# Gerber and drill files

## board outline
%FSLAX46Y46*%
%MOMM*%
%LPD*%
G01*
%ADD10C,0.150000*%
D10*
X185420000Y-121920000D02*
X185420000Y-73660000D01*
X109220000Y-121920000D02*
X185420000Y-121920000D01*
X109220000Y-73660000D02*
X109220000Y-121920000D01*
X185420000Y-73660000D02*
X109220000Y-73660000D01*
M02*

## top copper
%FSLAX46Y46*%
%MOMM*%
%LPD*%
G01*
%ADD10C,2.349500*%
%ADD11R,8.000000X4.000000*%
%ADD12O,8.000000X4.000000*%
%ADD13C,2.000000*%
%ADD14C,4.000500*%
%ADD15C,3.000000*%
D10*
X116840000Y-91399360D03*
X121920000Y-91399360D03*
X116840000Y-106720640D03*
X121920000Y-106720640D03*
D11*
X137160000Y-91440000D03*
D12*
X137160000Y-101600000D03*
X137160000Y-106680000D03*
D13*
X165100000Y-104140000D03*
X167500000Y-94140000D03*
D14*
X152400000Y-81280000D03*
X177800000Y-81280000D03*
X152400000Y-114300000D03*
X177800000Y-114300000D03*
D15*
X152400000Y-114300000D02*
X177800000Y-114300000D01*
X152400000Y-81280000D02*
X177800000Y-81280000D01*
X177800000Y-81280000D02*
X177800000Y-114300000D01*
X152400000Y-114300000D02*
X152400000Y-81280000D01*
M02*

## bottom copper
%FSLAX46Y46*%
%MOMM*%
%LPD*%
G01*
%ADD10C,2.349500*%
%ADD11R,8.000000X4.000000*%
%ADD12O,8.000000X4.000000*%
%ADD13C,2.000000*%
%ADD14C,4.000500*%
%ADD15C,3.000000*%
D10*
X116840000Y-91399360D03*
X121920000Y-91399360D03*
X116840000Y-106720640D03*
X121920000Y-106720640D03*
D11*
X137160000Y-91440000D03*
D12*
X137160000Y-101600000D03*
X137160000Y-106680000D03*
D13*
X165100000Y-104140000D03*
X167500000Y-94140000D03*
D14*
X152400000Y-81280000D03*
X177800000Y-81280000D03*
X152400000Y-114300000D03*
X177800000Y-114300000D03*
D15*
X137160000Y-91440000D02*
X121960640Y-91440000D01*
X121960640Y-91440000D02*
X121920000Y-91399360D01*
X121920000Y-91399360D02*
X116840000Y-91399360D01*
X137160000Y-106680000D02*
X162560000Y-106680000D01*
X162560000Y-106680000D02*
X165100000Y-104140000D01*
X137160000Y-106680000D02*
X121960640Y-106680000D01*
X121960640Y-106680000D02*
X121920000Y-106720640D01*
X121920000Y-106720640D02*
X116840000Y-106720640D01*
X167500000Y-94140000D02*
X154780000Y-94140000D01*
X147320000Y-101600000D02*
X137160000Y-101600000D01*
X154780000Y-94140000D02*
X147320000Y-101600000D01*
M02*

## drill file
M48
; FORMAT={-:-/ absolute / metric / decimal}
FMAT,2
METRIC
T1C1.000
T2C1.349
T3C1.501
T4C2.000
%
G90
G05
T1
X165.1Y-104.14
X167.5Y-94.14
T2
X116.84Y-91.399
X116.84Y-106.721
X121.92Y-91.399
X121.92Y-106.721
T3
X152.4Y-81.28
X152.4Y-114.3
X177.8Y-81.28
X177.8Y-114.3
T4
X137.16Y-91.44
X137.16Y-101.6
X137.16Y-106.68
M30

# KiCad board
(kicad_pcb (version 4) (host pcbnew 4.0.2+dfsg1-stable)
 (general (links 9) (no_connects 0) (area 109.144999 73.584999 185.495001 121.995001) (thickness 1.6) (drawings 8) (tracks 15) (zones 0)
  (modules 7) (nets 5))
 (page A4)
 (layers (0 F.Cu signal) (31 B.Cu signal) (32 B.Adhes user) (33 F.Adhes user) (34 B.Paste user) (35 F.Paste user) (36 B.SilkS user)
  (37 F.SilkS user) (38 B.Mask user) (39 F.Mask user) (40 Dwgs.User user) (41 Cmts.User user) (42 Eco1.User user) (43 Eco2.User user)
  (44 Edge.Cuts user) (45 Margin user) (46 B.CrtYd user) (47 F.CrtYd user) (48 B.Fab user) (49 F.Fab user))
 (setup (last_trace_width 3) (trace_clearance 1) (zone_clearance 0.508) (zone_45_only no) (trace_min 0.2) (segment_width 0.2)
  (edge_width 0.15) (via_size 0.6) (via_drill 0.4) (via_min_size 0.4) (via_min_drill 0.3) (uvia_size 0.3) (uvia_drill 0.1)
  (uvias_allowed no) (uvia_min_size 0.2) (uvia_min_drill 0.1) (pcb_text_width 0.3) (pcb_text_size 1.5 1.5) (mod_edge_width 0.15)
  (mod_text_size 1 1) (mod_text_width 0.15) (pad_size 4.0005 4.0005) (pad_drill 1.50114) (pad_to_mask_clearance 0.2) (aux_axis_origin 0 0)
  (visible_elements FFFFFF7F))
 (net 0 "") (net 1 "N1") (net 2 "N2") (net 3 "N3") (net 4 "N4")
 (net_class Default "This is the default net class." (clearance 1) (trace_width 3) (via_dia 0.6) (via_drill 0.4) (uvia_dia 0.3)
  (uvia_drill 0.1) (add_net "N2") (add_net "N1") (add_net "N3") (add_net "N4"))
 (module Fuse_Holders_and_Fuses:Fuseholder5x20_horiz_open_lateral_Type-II (layer F.Cu) (at 119.38 99.06 90)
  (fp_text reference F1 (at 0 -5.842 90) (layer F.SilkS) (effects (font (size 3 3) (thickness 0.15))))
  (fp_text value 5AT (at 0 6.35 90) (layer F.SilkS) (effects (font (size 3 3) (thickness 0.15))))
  (pad 2 thru_hole circle (at 7.66064 -2.54 90) (size 2.3495 2.3495) (drill 1.34874) (layers *.Cu *.Mask F.SilkS) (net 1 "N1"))
  (pad 2 thru_hole circle (at 7.66064 2.54 90) (size 2.3495 2.3495) (drill 1.34874) (layers *.Cu *.Mask F.SilkS) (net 1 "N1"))
  (pad 1 thru_hole circle (at -7.66064 -2.54 90) (size 2.3495 2.3495) (drill 1.34874) (layers *.Cu *.Mask F.SilkS) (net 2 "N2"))
  (pad 1 thru_hole circle (at -7.66064 2.54 90) (size 2.3495 2.3495) (drill 1.34874) (layers *.Cu *.Mask F.SilkS) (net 2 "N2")))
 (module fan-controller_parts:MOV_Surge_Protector (layer F.Cu) (at 137.16 91.44)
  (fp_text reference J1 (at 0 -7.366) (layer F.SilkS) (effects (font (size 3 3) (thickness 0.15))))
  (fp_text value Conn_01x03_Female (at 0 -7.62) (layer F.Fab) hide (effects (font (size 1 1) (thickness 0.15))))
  (pad 1 thru_hole rect (at 0 0) (size 8 4) (drill 2) (layers *.Cu *.Mask F.SilkS) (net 1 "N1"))
  (pad 2 thru_hole oval (at 0 10.16) (size 8 4) (drill 2) (layers *.Cu *.Mask F.SilkS) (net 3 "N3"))
  (pad 3 thru_hole oval (at 0 15.24) (size 8 4) (drill 2) (layers *.Cu *.Mask F.SilkS) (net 2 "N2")))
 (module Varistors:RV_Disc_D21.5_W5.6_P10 (layer F.Cu) (at 165.1 104.14 90)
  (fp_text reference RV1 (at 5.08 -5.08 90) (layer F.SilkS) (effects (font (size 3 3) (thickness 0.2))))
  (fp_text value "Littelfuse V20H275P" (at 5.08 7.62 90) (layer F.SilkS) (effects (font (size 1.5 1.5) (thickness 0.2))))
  (pad 1 thru_hole circle (at 0 0 90) (size 2 2) (drill 1) (layers *.Cu *.Mask F.SilkS) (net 2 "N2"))
  (pad 2 thru_hole circle (at 10 2.4 90) (size 2 2) (drill 1) (layers *.Cu *.Mask F.SilkS) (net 3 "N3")))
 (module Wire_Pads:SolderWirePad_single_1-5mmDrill (layer F.Cu) (at 152.4 81.28)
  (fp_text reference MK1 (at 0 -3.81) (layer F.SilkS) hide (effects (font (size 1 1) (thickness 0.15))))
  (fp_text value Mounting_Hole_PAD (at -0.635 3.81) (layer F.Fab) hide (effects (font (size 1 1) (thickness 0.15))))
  (pad 1 thru_hole circle (at 0 0) (size 4.0005 4.0005) (drill 1.50114) (layers *.Cu *.Mask F.SilkS) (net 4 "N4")))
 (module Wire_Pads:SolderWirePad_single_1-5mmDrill (layer F.Cu) (at 177.8 81.28)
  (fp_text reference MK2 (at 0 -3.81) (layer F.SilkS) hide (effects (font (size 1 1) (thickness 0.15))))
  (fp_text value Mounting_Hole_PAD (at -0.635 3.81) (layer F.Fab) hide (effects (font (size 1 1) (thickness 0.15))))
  (pad 1 thru_hole circle (at 0 0) (size 4.0005 4.0005) (drill 1.50114) (layers *.Cu *.Mask F.SilkS) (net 4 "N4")))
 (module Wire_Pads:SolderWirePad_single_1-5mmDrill (layer F.Cu) (at 152.4 114.3)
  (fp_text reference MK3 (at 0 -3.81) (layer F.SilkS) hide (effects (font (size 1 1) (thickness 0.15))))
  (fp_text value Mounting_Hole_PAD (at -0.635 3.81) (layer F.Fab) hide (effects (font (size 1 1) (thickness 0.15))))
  (pad 1 thru_hole circle (at 0 0) (size 4.0005 4.0005) (drill 1.50114) (layers *.Cu *.Mask F.SilkS) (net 4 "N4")))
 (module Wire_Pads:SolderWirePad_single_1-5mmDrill (layer F.Cu) (at 177.8 114.3)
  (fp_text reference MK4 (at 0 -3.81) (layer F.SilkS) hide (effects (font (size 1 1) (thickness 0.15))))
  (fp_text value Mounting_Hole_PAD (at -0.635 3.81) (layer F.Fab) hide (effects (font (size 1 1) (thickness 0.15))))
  (pad 1 thru_hole circle (at 0 0) (size 4.0005 4.0005) (drill 1.50114) (layers *.Cu *.Mask F.SilkS) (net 4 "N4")))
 (gr_line (start 185.42 121.92) (end 185.42 73.66) (angle 90) (layer Edge.Cuts) (width 0.15))
 (gr_line (start 109.22 121.92) (end 185.42 121.92) (angle 90) (layer Edge.Cuts) (width 0.15))
 (gr_line (start 109.22 73.66) (end 109.22 121.92) (angle 90) (layer Edge.Cuts) (width 0.15))
 (gr_line (start 185.42 73.66) (end 109.22 73.66) (angle 90) (layer Edge.Cuts) (width 0.15))
 (segment (start 137.16 91.44) (end 121.96064 91.44) (width 3) (layer B.Cu) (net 1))
 (segment (start 121.96064 91.44) (end 121.92 91.39936) (width 3) (layer B.Cu) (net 1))
 (segment (start 121.92 91.39936) (end 116.84 91.39936) (width 3) (layer B.Cu) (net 1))
 (segment (start 137.16 106.68) (end 162.56 106.68) (width 3) (layer B.Cu) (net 2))
 (segment (start 162.56 106.68) (end 165.1 104.14) (width 3) (layer B.Cu) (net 2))
 (segment (start 137.16 106.68) (end 121.96064 106.68) (width 3) (layer B.Cu) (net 2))
 (segment (start 121.96064 106.68) (end 121.92 106.72064) (width 3) (layer B.Cu) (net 2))
 (segment (start 121.92 106.72064) (end 116.84 106.72064) (width 3) (layer B.Cu) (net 2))
 (segment (start 167.5 94.14) (end 154.78 94.14) (width 3) (layer B.Cu) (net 3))
 (segment (start 147.32 101.6) (end 137.16 101.6) (width 3) (layer B.Cu) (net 3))
 (segment (start 154.78 94.14) (end 147.32 101.6) (width 3) (layer B.Cu) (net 3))
 (segment (start 152.4 114.3) (end 177.8 114.3) (width 3) (layer F.Cu) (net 4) (status C00000))
 (segment (start 152.4 81.28) (end 177.8 81.28) (width 3) (layer F.Cu) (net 4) (status C00000))
 (segment (start 177.8 81.28) (end 177.8 114.3) (width 3) (layer F.Cu) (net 4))
 (segment (start 152.4 114.3) (end 152.4 81.28) (width 3) (layer F.Cu) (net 4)))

